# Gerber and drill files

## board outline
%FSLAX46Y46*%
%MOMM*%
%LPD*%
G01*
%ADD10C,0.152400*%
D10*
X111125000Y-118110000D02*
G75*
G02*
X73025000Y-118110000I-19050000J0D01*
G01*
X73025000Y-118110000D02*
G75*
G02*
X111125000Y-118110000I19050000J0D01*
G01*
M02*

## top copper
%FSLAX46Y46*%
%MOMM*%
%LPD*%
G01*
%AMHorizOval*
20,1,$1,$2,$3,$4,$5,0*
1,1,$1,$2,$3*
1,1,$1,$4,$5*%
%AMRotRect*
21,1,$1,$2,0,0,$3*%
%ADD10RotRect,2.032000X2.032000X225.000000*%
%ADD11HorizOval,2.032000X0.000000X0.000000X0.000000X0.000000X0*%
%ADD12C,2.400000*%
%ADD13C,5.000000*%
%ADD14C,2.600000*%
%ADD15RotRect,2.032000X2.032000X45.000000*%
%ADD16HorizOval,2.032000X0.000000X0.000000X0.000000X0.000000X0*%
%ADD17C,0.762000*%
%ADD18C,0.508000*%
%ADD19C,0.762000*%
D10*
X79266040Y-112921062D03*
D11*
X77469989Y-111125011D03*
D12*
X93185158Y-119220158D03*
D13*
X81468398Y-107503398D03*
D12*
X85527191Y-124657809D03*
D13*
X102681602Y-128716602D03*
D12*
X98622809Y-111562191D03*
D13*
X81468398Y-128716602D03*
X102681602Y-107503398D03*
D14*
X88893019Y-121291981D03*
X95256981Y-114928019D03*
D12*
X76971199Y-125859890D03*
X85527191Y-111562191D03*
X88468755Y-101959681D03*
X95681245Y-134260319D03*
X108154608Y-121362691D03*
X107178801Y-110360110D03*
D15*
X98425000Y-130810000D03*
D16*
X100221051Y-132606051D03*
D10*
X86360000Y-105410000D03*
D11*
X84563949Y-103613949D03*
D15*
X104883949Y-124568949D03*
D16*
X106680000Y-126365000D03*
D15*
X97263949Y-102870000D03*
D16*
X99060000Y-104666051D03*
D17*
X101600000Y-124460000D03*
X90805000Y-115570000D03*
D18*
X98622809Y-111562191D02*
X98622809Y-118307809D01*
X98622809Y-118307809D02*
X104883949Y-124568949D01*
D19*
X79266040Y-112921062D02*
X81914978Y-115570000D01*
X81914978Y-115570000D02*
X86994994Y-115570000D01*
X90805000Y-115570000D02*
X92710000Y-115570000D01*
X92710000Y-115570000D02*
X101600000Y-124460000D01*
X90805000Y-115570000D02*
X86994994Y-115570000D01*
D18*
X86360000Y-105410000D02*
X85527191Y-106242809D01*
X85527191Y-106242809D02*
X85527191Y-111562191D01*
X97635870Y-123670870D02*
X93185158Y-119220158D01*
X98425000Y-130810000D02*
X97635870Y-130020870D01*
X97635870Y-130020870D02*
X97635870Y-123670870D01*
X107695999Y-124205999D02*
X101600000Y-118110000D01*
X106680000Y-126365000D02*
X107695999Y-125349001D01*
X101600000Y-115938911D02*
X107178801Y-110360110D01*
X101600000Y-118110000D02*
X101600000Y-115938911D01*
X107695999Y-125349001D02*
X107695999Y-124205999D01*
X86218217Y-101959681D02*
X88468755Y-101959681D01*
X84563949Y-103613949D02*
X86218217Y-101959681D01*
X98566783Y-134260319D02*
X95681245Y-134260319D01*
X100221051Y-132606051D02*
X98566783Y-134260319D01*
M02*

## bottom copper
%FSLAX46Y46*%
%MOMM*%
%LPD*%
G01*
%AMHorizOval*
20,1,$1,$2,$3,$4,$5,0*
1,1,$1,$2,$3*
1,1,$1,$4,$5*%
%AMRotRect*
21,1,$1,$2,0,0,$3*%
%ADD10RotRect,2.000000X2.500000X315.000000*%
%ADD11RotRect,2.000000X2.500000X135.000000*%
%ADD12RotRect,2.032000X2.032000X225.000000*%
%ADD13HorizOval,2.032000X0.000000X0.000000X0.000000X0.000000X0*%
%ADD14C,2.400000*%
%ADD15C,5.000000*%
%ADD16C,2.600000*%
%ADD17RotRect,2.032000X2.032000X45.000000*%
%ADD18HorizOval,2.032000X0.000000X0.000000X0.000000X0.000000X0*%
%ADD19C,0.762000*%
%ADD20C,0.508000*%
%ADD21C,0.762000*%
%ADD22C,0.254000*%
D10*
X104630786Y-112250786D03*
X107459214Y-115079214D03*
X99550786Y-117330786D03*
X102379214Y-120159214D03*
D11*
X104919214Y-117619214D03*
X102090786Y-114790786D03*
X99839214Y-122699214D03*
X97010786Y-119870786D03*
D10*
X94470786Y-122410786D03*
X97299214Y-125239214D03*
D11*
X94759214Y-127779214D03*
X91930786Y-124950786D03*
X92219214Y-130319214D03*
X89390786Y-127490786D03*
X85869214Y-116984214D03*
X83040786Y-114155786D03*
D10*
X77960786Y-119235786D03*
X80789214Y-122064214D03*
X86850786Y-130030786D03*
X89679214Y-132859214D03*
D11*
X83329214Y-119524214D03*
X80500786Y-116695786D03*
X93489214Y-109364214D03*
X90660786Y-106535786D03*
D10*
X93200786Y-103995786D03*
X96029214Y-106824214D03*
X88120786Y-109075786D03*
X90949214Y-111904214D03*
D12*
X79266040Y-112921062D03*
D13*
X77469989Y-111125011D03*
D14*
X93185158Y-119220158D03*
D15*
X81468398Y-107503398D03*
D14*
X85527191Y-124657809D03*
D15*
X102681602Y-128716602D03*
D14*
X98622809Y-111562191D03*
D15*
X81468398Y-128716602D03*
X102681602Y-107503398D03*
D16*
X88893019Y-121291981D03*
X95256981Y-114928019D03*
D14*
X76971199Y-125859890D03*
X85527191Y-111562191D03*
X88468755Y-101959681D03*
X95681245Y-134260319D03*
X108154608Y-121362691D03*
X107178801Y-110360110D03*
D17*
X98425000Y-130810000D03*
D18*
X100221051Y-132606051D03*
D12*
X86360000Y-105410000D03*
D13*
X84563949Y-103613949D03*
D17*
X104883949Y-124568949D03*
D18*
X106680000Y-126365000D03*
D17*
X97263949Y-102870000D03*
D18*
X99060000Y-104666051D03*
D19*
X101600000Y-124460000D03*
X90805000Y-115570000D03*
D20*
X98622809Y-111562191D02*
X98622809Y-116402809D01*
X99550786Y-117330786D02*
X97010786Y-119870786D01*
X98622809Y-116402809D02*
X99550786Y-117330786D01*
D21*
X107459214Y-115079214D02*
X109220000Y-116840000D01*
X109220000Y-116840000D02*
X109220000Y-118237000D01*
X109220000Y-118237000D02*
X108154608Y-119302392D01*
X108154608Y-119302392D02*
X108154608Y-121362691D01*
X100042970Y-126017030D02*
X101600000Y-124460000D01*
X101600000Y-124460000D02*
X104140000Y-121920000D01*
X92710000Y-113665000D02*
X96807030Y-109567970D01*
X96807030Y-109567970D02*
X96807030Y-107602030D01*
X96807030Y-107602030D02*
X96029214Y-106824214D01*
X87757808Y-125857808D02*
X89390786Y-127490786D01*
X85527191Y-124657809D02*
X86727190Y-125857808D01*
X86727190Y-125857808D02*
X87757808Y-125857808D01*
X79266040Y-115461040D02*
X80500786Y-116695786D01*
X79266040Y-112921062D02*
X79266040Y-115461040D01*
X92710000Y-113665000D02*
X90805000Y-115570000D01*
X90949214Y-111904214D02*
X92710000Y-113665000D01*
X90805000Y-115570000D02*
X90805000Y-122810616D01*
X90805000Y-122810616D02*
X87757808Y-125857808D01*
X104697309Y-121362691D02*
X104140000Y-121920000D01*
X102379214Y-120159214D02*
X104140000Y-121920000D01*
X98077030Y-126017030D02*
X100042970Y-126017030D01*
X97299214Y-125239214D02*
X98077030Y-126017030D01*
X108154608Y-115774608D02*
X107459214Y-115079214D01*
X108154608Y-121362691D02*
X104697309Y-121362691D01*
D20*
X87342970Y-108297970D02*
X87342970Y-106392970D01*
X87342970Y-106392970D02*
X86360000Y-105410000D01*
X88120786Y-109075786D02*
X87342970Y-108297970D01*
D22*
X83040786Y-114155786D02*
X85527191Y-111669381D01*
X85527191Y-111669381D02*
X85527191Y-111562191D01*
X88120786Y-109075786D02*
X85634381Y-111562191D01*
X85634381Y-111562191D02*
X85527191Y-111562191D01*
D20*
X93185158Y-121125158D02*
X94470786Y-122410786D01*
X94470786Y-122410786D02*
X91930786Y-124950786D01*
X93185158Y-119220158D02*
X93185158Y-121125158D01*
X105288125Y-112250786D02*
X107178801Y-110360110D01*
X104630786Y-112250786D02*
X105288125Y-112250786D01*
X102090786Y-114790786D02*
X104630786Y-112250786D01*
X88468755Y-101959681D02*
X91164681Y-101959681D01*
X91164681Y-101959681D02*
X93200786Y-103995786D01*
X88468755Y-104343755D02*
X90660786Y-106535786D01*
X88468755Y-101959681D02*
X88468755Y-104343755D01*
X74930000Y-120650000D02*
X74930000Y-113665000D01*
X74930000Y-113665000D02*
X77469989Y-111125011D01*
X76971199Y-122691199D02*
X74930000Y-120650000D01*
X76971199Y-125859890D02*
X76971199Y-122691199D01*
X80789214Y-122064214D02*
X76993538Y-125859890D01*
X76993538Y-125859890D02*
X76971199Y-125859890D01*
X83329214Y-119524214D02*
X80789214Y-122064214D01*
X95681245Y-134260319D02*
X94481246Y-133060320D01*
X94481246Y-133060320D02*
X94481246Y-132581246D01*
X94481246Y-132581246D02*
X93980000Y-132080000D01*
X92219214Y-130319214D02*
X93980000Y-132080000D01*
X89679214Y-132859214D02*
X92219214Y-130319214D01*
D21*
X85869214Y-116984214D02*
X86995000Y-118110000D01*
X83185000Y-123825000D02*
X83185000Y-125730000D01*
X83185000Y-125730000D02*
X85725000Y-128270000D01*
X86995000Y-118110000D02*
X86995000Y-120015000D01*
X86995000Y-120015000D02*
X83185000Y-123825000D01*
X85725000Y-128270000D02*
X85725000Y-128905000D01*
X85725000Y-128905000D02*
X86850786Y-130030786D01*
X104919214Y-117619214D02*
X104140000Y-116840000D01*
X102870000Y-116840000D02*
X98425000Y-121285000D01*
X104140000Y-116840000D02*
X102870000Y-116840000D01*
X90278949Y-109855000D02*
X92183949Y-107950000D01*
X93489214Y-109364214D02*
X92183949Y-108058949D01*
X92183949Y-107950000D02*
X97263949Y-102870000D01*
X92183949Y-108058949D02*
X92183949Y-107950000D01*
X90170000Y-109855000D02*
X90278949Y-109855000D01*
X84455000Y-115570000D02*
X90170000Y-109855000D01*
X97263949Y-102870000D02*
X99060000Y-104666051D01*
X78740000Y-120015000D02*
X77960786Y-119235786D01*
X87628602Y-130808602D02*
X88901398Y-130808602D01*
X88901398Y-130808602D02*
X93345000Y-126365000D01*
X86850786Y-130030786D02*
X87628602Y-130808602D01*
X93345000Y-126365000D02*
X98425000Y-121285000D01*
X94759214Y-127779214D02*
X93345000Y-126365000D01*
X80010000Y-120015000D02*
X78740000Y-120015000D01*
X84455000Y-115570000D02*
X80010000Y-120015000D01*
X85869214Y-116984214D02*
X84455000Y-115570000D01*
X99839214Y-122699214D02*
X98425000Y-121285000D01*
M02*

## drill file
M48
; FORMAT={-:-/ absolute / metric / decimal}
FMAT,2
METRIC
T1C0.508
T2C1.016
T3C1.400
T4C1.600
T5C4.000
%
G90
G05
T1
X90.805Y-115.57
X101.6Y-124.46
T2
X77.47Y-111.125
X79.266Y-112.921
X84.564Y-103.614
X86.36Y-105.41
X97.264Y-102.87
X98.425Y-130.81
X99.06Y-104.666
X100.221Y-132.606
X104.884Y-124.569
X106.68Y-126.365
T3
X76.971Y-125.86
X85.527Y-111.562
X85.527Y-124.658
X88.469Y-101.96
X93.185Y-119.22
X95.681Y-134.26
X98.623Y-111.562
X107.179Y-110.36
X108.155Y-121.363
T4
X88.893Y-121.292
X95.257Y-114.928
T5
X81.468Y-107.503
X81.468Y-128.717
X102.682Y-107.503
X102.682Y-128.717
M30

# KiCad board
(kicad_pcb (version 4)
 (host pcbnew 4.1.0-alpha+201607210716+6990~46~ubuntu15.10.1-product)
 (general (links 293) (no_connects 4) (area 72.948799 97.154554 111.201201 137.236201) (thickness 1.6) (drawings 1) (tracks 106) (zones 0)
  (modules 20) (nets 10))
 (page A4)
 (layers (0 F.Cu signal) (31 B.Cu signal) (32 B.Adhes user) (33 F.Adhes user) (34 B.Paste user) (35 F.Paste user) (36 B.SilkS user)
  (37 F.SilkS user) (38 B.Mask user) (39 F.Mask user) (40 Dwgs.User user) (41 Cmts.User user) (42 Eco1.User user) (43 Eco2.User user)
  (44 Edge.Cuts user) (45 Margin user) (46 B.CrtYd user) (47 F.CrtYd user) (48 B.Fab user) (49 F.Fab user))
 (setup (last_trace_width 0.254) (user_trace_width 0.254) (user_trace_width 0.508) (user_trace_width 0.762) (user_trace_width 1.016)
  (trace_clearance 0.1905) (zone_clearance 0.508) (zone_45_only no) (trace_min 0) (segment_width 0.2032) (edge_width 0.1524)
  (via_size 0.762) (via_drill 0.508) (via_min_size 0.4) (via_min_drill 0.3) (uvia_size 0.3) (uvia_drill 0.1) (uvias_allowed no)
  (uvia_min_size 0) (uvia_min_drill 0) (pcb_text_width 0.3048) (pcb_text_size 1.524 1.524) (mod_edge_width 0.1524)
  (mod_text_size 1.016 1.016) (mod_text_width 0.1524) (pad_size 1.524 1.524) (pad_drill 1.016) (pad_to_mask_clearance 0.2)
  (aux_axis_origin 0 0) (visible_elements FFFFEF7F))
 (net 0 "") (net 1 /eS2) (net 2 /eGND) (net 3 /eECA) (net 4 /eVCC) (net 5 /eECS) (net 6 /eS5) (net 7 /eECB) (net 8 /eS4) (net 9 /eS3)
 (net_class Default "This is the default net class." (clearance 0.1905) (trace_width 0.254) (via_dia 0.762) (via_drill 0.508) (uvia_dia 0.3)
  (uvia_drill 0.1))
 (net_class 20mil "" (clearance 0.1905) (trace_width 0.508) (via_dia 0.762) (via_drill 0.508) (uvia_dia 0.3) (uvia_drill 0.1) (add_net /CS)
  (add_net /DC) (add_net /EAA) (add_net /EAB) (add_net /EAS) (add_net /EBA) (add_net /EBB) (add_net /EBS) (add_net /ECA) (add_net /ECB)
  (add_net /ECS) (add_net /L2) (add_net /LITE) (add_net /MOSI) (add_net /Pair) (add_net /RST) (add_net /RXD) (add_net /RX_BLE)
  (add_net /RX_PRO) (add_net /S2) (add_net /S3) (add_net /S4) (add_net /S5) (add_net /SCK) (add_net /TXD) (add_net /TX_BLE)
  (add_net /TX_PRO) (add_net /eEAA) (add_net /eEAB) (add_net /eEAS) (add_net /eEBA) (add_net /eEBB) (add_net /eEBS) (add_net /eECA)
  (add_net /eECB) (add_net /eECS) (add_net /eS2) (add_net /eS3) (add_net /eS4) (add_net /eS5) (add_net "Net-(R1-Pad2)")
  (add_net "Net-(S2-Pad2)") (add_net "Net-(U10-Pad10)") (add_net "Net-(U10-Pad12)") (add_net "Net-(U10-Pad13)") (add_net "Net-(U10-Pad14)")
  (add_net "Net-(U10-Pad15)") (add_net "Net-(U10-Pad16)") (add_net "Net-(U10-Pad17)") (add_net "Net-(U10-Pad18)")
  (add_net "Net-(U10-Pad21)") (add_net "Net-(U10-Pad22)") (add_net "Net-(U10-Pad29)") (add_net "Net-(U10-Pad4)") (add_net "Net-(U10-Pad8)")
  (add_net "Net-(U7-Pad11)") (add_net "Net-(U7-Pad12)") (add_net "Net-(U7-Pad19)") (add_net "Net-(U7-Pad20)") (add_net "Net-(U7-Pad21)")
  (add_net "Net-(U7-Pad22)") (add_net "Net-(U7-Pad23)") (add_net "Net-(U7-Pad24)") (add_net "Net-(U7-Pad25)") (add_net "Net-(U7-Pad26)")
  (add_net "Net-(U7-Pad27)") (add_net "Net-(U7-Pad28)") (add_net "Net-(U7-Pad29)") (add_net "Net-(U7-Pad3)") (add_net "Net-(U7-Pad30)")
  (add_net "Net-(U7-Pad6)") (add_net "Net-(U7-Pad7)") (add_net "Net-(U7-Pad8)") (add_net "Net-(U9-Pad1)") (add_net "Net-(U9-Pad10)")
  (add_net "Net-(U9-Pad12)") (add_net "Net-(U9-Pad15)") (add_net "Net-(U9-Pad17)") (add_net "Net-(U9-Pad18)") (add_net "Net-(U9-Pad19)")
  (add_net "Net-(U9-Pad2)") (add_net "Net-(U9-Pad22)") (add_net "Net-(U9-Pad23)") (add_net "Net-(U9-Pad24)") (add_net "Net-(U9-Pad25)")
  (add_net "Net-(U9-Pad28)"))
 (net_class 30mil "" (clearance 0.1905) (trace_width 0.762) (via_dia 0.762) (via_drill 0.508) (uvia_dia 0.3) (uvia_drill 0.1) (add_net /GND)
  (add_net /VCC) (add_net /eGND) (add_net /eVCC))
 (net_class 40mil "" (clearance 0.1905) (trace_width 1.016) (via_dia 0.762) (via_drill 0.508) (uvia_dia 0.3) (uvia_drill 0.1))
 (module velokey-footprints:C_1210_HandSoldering (layer B.Cu) (at 106.045 113.665 315)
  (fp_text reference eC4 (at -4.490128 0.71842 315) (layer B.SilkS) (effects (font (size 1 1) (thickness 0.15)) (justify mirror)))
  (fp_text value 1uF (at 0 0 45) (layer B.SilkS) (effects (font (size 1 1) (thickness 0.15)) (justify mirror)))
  (pad 1 smd rect (at -2 0 315) (size 2 2.5) (layers B.Cu B.Paste B.Mask) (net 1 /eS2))
  (pad 2 smd rect (at 2 0 315) (size 2 2.5) (layers B.Cu B.Paste B.Mask) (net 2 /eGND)))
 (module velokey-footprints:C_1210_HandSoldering (layer B.Cu) (at 100.965 118.745 315)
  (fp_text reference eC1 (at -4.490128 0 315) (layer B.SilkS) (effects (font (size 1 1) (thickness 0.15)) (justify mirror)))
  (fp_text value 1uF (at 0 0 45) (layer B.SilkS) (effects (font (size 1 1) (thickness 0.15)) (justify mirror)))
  (pad 1 smd rect (at -2 0 315) (size 2 2.5) (layers B.Cu B.Paste B.Mask) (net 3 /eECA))
  (pad 2 smd rect (at 2 0 315) (size 2 2.5) (layers B.Cu B.Paste B.Mask) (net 2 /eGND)))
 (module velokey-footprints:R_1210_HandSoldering (layer B.Cu) (at 103.505 116.205 135)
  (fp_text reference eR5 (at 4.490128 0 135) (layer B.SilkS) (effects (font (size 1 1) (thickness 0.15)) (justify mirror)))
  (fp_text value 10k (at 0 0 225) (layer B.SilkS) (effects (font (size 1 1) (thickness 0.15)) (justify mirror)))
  (pad 1 smd rect (at -2 0 135) (size 2 2.5) (layers B.Cu B.Paste B.Mask) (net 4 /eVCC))
  (pad 2 smd rect (at 2 0 135) (size 2 2.5) (layers B.Cu B.Paste B.Mask) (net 1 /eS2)))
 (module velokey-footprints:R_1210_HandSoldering (layer B.Cu) (at 98.425 121.285 135)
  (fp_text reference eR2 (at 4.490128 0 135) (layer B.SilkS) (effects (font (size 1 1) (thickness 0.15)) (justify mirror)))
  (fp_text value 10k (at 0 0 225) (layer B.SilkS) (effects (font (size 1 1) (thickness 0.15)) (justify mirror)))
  (pad 1 smd rect (at -2 0 135) (size 2 2.5) (layers B.Cu B.Paste B.Mask) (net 4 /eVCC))
  (pad 2 smd rect (at 2 0 135) (size 2 2.5) (layers B.Cu B.Paste B.Mask) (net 3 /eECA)))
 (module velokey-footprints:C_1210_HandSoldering (layer B.Cu) (at 95.885 123.825 315)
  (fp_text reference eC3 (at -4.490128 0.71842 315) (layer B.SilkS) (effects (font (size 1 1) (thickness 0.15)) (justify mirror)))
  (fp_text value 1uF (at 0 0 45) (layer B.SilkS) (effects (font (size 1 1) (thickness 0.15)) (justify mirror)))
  (pad 1 smd rect (at -2 0 315) (size 2 2.5) (layers B.Cu B.Paste B.Mask) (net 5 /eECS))
  (pad 2 smd rect (at 2 0 315) (size 2 2.5) (layers B.Cu B.Paste B.Mask) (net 2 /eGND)))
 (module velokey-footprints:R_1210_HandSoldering (layer B.Cu) (at 93.345 126.365 135)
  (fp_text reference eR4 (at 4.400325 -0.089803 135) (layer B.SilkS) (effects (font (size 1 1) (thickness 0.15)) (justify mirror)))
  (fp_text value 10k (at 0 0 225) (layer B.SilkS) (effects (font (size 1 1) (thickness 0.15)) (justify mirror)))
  (pad 1 smd rect (at -2 0 135) (size 2 2.5) (layers B.Cu B.Paste B.Mask) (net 4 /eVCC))
  (pad 2 smd rect (at 2 0 135) (size 2 2.5) (layers B.Cu B.Paste B.Mask) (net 5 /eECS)))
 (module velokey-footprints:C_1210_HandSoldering (layer B.Cu) (at 90.805 128.905 135)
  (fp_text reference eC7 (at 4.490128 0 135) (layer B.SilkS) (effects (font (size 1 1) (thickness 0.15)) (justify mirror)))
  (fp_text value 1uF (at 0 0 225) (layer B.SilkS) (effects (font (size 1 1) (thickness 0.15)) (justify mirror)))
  (pad 1 smd rect (at -2 0 135) (size 2 2.5) (layers B.Cu B.Paste B.Mask) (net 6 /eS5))
  (pad 2 smd rect (at 2 0 135) (size 2 2.5) (layers B.Cu B.Paste B.Mask) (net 2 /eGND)))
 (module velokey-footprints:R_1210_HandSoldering (layer B.Cu) (at 84.455 115.57 135)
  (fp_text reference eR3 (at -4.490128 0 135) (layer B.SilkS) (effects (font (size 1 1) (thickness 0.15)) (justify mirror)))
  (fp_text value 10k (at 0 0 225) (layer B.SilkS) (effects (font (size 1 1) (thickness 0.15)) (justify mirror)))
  (pad 1 smd rect (at -2 0 135) (size 2 2.5) (layers B.Cu B.Paste B.Mask) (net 4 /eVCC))
  (pad 2 smd rect (at 2 0 135) (size 2 2.5) (layers B.Cu B.Paste B.Mask) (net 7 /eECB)))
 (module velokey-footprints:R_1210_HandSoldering (layer B.Cu) (at 79.375 120.65 315)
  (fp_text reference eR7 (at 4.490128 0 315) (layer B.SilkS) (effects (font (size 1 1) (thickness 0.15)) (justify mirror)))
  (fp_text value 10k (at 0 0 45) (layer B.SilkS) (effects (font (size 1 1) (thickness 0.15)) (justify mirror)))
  (pad 1 smd rect (at -2 0 315) (size 2 2.5) (layers B.Cu B.Paste B.Mask) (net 4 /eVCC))
  (pad 2 smd rect (at 2 0 315) (size 2 2.5) (layers B.Cu B.Paste B.Mask) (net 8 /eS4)))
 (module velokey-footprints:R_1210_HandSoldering (layer B.Cu) (at 88.265 131.445 315)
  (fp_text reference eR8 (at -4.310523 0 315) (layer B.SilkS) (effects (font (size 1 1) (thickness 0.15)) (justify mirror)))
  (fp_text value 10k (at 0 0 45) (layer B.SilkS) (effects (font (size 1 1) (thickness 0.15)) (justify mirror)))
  (pad 1 smd rect (at -2 0 315) (size 2 2.5) (layers B.Cu B.Paste B.Mask) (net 4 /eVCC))
  (pad 2 smd rect (at 2 0 315) (size 2 2.5) (layers B.Cu B.Paste B.Mask) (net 6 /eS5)))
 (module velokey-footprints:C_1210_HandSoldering (layer B.Cu) (at 81.915 118.11 135)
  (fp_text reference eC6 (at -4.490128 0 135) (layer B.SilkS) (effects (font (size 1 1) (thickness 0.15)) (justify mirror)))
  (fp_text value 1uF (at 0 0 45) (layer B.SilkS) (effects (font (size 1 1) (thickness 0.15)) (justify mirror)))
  (pad 1 smd rect (at -2 0 135) (size 2 2.5) (layers B.Cu B.Paste B.Mask) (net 8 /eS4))
  (pad 2 smd rect (at 2 0 135) (size 2 2.5) (layers B.Cu B.Paste B.Mask) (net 2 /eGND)))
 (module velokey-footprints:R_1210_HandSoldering (layer B.Cu) (at 92.075 107.95 135)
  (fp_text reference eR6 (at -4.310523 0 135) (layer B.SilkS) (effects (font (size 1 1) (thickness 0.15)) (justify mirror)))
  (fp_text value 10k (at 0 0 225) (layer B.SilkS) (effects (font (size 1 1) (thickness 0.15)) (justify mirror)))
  (pad 1 smd rect (at -2 0 135) (size 2 2.5) (layers B.Cu B.Paste B.Mask) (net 4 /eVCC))
  (pad 2 smd rect (at 2 0 135) (size 2 2.5) (layers B.Cu B.Paste B.Mask) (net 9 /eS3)))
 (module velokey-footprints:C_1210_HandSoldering (layer B.Cu) (at 94.615 105.41 315)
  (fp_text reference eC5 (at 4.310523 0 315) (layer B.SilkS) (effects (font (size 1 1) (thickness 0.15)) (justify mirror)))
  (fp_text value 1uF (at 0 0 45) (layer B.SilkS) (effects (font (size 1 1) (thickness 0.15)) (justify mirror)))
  (pad 1 smd rect (at -2 0 315) (size 2 2.5) (layers B.Cu B.Paste B.Mask) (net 9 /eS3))
  (pad 2 smd rect (at 2 0 315) (size 2 2.5) (layers B.Cu B.Paste B.Mask) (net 2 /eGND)))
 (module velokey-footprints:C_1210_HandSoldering (layer B.Cu) (at 89.535 110.49 315)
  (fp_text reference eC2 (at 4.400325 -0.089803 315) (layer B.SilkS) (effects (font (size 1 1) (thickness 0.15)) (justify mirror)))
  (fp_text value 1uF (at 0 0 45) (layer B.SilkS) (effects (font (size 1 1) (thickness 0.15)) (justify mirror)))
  (pad 1 smd rect (at -2 0 315) (size 2 2.5) (layers B.Cu B.Paste B.Mask) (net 7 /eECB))
  (pad 2 smd rect (at 2 0 315) (size 2 2.5) (layers B.Cu B.Paste B.Mask) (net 2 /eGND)))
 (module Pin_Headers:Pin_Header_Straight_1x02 (layer F.Cu) (at 79.26604 112.921062 225)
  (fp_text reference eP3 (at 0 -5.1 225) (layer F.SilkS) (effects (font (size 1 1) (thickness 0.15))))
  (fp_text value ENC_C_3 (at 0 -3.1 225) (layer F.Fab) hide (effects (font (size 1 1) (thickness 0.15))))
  (pad 1 thru_hole rect (at 0 0 225) (size 2.032 2.032) (drill 1.016) (layers *.Cu *.Mask F.SilkS) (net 2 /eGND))
  (pad 2 thru_hole oval (at 0 2.54 225) (size 2.032 2.032) (drill 1.016) (layers *.Cu *.Mask F.SilkS) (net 8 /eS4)))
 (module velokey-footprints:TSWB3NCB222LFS (layer F.Cu) (at 92.075 118.11 45)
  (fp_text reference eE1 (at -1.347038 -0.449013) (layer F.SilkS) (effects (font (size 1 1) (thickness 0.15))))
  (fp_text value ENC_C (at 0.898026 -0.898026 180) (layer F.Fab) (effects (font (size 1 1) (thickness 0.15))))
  (pad 4 thru_hole circle (at 0 1.57 45) (size 2.4 2.4) (drill 1.4) (layers *.Cu *.Mask F.SilkS) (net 5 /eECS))
  (pad 12 thru_hole circle (at 0 -15 45) (size 5 5) (drill 4) (layers *.Cu *.Mask F.SilkS))
  (pad 2 thru_hole circle (at -9.26 0 45) (size 2.4 2.4) (drill 1.4) (layers *.Cu *.Mask F.SilkS) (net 2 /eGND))
  (pad 14 thru_hole circle (at 0 15 45) (size 5 5) (drill 4) (layers *.Cu *.Mask F.SilkS))
  (pad 1 thru_hole circle (at 9.26 0 45) (size 2.4 2.4) (drill 1.4) (layers *.Cu *.Mask F.SilkS) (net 3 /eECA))
  (pad 13 thru_hole circle (at -15 0 45) (size 5 5) (drill 4) (layers *.Cu *.Mask F.SilkS))
  (pad 15 thru_hole circle (at 15 0 45) (size 5 5) (drill 4) (layers *.Cu *.Mask F.SilkS))
  (pad 5 thru_hole circle (at -4.5 0 45) (size 2.6 2.6) (drill 1.6) (layers *.Cu *.Mask F.SilkS))
  (pad 6 thru_hole circle (at 4.5 0 45) (size 2.6 2.6) (drill 1.6) (layers *.Cu *.Mask F.SilkS))
  (pad 9 thru_hole circle (at -16.16 -5.2 45) (size 2.4 2.4) (drill 1.4) (layers *.Cu *.Mask F.SilkS) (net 8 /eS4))
  (pad 3 thru_hole circle (at 0 -9.26 45) (size 2.4 2.4) (drill 1.4) (layers *.Cu *.Mask F.SilkS) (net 7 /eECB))
  (pad 8 thru_hole circle (at 8.87 -13.97 45) (size 2.4 2.4) (drill 1.4) (layers *.Cu *.Mask F.SilkS) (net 9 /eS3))
  (pad 10 thru_hole circle (at -8.87 13.97 45) (size 2.4 2.4) (drill 1.4) (layers *.Cu *.Mask F.SilkS) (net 6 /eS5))
  (pad 11 thru_hole circle (at 9.07 13.67 45) (size 2.4 2.4) (drill 1.4) (layers *.Cu *.Mask F.SilkS) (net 2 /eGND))
  (pad 7 thru_hole circle (at 16.16 5.2 45) (size 2.4 2.4) (drill 1.4) (layers *.Cu *.Mask F.SilkS) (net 1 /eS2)))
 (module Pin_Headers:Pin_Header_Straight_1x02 (layer F.Cu) (at 98.425 130.81 45)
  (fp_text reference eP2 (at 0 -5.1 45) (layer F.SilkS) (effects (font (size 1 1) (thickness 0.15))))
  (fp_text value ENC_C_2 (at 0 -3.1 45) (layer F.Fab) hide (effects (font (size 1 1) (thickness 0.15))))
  (pad 1 thru_hole rect (at 0 0 45) (size 2.032 2.032) (drill 1.016) (layers *.Cu *.Mask F.SilkS) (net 5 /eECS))
  (pad 2 thru_hole oval (at 0 2.54 45) (size 2.032 2.032) (drill 1.016) (layers *.Cu *.Mask F.SilkS) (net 6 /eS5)))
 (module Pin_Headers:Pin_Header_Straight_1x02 (layer F.Cu) (at 86.36 105.41 225)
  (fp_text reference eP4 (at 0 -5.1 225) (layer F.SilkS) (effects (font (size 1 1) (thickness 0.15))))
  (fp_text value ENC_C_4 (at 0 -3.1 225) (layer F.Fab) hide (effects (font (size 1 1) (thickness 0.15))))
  (pad 1 thru_hole rect (at 0 0 225) (size 2.032 2.032) (drill 1.016) (layers *.Cu *.Mask F.SilkS) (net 7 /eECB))
  (pad 2 thru_hole oval (at 0 2.54 225) (size 2.032 2.032) (drill 1.016) (layers *.Cu *.Mask F.SilkS) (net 9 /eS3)))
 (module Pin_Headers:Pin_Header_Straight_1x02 (layer F.Cu) (at 104.883949 124.568949 45)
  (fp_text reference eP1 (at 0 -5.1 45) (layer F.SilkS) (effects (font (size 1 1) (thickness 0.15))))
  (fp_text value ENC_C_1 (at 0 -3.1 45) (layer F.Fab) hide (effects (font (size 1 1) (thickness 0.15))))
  (pad 1 thru_hole rect (at 0 0 45) (size 2.032 2.032) (drill 1.016) (layers *.Cu *.Mask F.SilkS) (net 3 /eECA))
  (pad 2 thru_hole oval (at 0 2.54 45) (size 2.032 2.032) (drill 1.016) (layers *.Cu *.Mask F.SilkS) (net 1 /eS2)))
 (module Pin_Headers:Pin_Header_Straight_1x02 (layer F.Cu) (at 97.263949 102.87 45)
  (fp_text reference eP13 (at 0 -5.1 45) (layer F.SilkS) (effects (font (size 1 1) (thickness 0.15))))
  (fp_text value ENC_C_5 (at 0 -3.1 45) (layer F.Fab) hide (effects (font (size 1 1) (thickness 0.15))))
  (pad 1 thru_hole rect (at 0 0 45) (size 2.032 2.032) (drill 1.016) (layers *.Cu *.Mask F.SilkS) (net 4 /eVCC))
  (pad 2 thru_hole oval (at 0 2.54 45) (size 2.032 2.032) (drill 1.016) (layers *.Cu *.Mask F.SilkS) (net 4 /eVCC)))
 (gr_circle (center 92.075 118.11) (end 111.125 118.11) (layer Edge.Cuts) (width 0.1524))
 (segment (start 98.622809 111.562191) (end 98.622809 116.402809) (width 0.508) (layer B.Cu) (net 3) (status 10))
 (segment (start 99.550786 117.330786) (end 97.010786 119.870786) (width 0.508) (layer B.Cu) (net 3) (status 30))
 (segment (start 98.622809 116.402809) (end 99.550786 117.330786) (width 0.508) (layer B.Cu) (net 3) (status 20))
 (segment (start 98.622809 111.562191) (end 98.622809 118.307809) (width 0.508) (layer F.Cu) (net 3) (status 10))
 (segment (start 98.622809 118.307809) (end 104.883949 124.568949) (width 0.508) (layer F.Cu) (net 3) (status 20))
 (segment (start 107.459214 115.079214) (end 109.22 116.84) (width 0.762) (layer B.Cu) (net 2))
 (segment (start 109.22 116.84) (end 109.22 118.237) (width 0.762) (layer B.Cu) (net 2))
 (segment (start 109.22 118.237) (end 108.154608 119.302392) (width 0.762) (layer B.Cu) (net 2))
 (segment (start 108.154608 119.302392) (end 108.154608 121.362691) (width 0.762) (layer B.Cu) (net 2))
 (segment (start 79.26604 112.921062) (end 81.914978 115.57) (width 0.762) (layer F.Cu) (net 2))
 (segment (start 81.914978 115.57) (end 86.994994 115.57) (width 0.762) (layer F.Cu) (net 2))
 (segment (start 100.04297 126.01703) (end 101.6 124.46) (width 0.762) (layer B.Cu) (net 2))
 (segment (start 101.6 124.46) (end 104.14 121.92) (width 0.762) (layer B.Cu) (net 2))
 (segment (start 90.805 115.57) (end 92.71 115.57) (width 0.762) (layer F.Cu) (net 2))
 (segment (start 92.71 115.57) (end 101.6 124.46) (width 0.762) (layer F.Cu) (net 2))
 (via (at 101.6 124.46) (size 0.762) (drill 0.508) (layers F.Cu B.Cu) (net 2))
 (segment (start 92.71 113.665) (end 96.80703 109.56797) (width 0.762) (layer B.Cu) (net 2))
 (segment (start 96.80703 109.56797) (end 96.80703 107.60203) (width 0.762) (layer B.Cu) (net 2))
 (segment (start 96.80703 107.60203) (end 96.029214 106.824214) (width 0.762) (layer B.Cu) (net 2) (status 20))
 (segment (start 87.757808 125.857808) (end 89.390786 127.490786) (width 0.762) (layer B.Cu) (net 2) (status 20))
 (segment (start 85.527191 124.657809) (end 86.72719 125.857808) (width 0.762) (layer B.Cu) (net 2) (status 10))
 (segment (start 86.72719 125.857808) (end 87.757808 125.857808) (width 0.762) (layer B.Cu) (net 2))
 (segment (start 79.26604 115.46104) (end 80.500786 116.695786) (width 0.762) (layer B.Cu) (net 2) (status 20))
 (segment (start 79.26604 112.921062) (end 79.26604 115.46104) (width 0.762) (layer B.Cu) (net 2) (status 10))
 (segment (start 92.71 113.665) (end 90.805 115.57) (width 0.762) (layer B.Cu) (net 2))
 (segment (start 90.949214 111.904214) (end 92.71 113.665) (width 0.762) (layer B.Cu) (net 2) (status 10))
 (segment (start 90.805 115.57) (end 90.805 122.810616) (width 0.762) (layer B.Cu) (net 2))
 (segment (start 90.805 122.810616) (end 87.757808 125.857808) (width 0.762) (layer B.Cu) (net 2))
 (segment (start 104.697309 121.362691) (end 104.14 121.92) (width 0.762) (layer B.Cu) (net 2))
 (segment (start 102.379214 120.159214) (end 104.14 121.92) (width 0.762) (layer B.Cu) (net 2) (status 10))
 (segment (start 98.07703 126.01703) (end 100.04297 126.01703) (width 0.762) (layer B.Cu) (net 2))
 (segment (start 97.299214 125.239214) (end 98.07703 126.01703) (width 0.762) (layer B.Cu) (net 2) (status 10))
 (segment (start 108.154608 115.774608) (end 107.459214 115.079214) (width 0.762) (layer B.Cu) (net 2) (status 30))
 (segment (start 108.154608 121.362691) (end 104.697309 121.362691) (width 0.762) (layer B.Cu) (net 2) (status 10))
 (segment (start 90.805 115.57) (end 86.994994 115.57) (width 0.762) (layer F.Cu) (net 2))
 (via (at 90.805 115.57) (size 0.762) (drill 0.508) (layers F.Cu B.Cu) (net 2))
 (segment (start 87.34297 108.29797) (end 87.34297 106.39297) (width 0.508) (layer B.Cu) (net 7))
 (segment (start 87.34297 106.39297) (end 86.36 105.41) (width 0.508) (layer B.Cu) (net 7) (status 20))
 (segment (start 88.120786 109.075786) (end 87.34297 108.29797) (width 0.508) (layer B.Cu) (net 7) (status 10))
 (segment (start 83.040786 114.155786) (end 85.527191 111.669381) (width 0.254) (layer B.Cu) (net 7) (status 30))
 (segment (start 85.527191 111.669381) (end 85.527191 111.562191) (width 0.254) (layer B.Cu) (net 7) (status 30))
 (segment (start 88.120786 109.075786) (end 85.634381 111.562191) (width 0.254) (layer B.Cu) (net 7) (status 30))
 (segment (start 85.634381 111.562191) (end 85.527191 111.562191) (width 0.254) (layer B.Cu) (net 7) (status 30))
 (segment (start 86.36 105.41) (end 85.527191 106.242809) (width 0.508) (layer F.Cu) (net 7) (status 10))
 (segment (start 85.527191 106.242809) (end 85.527191 111.562191) (width 0.508) (layer F.Cu) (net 7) (status 20))
 (segment (start 93.185158 121.125158) (end 94.470786 122.410786) (width 0.508) (layer B.Cu) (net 5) (status 20))
 (segment (start 94.470786 122.410786) (end 91.930786 124.950786) (width 0.508) (layer B.Cu) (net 5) (status 30))
 (segment (start 93.185158 119.220158) (end 93.185158 121.125158) (width 0.508) (layer B.Cu) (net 5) (status 10))
 (segment (start 97.63587 123.67087) (end 93.185158 119.220158) (width 0.508) (layer F.Cu) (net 5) (status 20))
 (segment (start 98.425 130.81) (end 97.63587 130.02087) (width 0.508) (layer F.Cu) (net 5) (status 10))
 (segment (start 97.63587 130.02087) (end 97.63587 123.67087) (width 0.508) (layer F.Cu) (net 5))
 (segment (start 105.288125 112.250786) (end 107.178801 110.36011) (width 0.508) (layer B.Cu) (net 1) (status 30))
 (segment (start 104.630786 112.250786) (end 105.288125 112.250786) (width 0.508) (layer B.Cu) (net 1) (status 30))
 (segment (start 102.090786 114.790786) (end 104.630786 112.250786) (width 0.508) (layer B.Cu) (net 1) (status 30))
 (segment (start 107.695999 124.205999) (end 101.6 118.11) (width 0.508) (layer F.Cu) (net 1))
 (segment (start 106.68 126.365) (end 107.695999 125.349001) (width 0.508) (layer F.Cu) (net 1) (status 10))
 (segment (start 101.6 115.938911) (end 107.178801 110.36011) (width 0.508) (layer F.Cu) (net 1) (status 20))
 (segment (start 101.6 118.11) (end 101.6 115.938911) (width 0.508) (layer F.Cu) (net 1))
 (segment (start 107.695999 125.349001) (end 107.695999 124.205999) (width 0.508) (layer F.Cu) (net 1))
 (segment (start 88.468755 101.959681) (end 91.164681 101.959681) (width 0.508) (layer B.Cu) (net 9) (status 10))
 (segment (start 91.164681 101.959681) (end 93.200786 103.995786) (width 0.508) (layer B.Cu) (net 9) (status 20))
 (segment (start 88.468755 104.343755) (end 90.660786 106.535786) (width 0.508) (layer B.Cu) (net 9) (status 20))
 (segment (start 88.468755 101.959681) (end 88.468755 104.343755) (width 0.508) (layer B.Cu) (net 9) (status 10))
 (segment (start 86.218217 101.959681) (end 88.468755 101.959681) (width 0.508) (layer F.Cu) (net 9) (status 20))
 (segment (start 84.563949 103.613949) (end 86.218217 101.959681) (width 0.508) (layer F.Cu) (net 9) (status 10))
 (segment (start 74.93 120.65) (end 74.93 113.665) (width 0.508) (layer B.Cu) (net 8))
 (segment (start 74.93 113.665) (end 77.469989 111.125011) (width 0.508) (layer B.Cu) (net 8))
 (segment (start 76.971199 122.691199) (end 74.93 120.65) (width 0.508) (layer B.Cu) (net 8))
 (segment (start 76.971199 125.85989) (end 76.971199 122.691199) (width 0.508) (layer B.Cu) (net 8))
 (segment (start 80.789214 122.064214) (end 76.993538 125.85989) (width 0.508) (layer B.Cu) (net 8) (status 30))
 (segment (start 76.993538 125.85989) (end 76.971199 125.85989) (width 0.508) (layer B.Cu) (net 8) (status 30))
 (segment (start 83.329214 119.524214) (end 80.789214 122.064214) (width 0.508) (layer B.Cu) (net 8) (status 30))
 (segment (start 95.681245 134.260319) (end 94.481246 133.06032) (width 0.508) (layer B.Cu) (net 6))
 (segment (start 94.481246 133.06032) (end 94.481246 132.581246) (width 0.508) (layer B.Cu) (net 6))
 (segment (start 94.481246 132.581246) (end 93.98 132.08) (width 0.508) (layer B.Cu) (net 6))
 (segment (start 92.219214 130.319214) (end 93.98 132.08) (width 0.508) (layer B.Cu) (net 6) (status 10))
 (segment (start 89.679214 132.859214) (end 92.219214 130.319214) (width 0.508) (layer B.Cu) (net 6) (status 30))
 (segment (start 98.566783 134.260319) (end 95.681245 134.260319) (width 0.508) (layer F.Cu) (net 6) (status 20))
 (segment (start 100.221051 132.606051) (end 98.566783 134.260319) (width 0.508) (layer F.Cu) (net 6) (status 10))
 (segment (start 85.869214 116.984214) (end 86.995 118.11) (width 0.762) (layer B.Cu) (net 4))
 (segment (start 83.185 123.825) (end 83.185 125.73) (width 0.762) (layer B.Cu) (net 4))
 (segment (start 83.185 125.73) (end 85.725 128.27) (width 0.762) (layer B.Cu) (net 4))
 (segment (start 86.995 118.11) (end 86.995 120.015) (width 0.762) (layer B.Cu) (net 4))
 (segment (start 86.995 120.015) (end 83.185 123.825) (width 0.762) (layer B.Cu) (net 4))
 (segment (start 85.725 128.27) (end 85.725 128.905) (width 0.762) (layer B.Cu) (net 4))
 (segment (start 85.725 128.905) (end 86.850786 130.030786) (width 0.762) (layer B.Cu) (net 4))
 (segment (start 104.919214 117.619214) (end 104.14 116.84) (width 0.762) (layer B.Cu) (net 4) (status 10))
 (segment (start 102.87 116.84) (end 98.425 121.285) (width 0.762) (layer B.Cu) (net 4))
 (segment (start 104.14 116.84) (end 102.87 116.84) (width 0.762) (layer B.Cu) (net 4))
 (segment (start 90.278949 109.855) (end 92.183949 107.95) (width 0.762) (layer B.Cu) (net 4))
 (segment (start 93.489214 109.364214) (end 92.183949 108.058949) (width 0.762) (layer B.Cu) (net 4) (status 10))
 (segment (start 92.183949 107.95) (end 97.263949 102.87) (width 0.762) (layer B.Cu) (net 4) (status 20))
 (segment (start 92.183949 108.058949) (end 92.183949 107.95) (width 0.762) (layer B.Cu) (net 4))
 (segment (start 90.17 109.855) (end 90.278949 109.855) (width 0.762) (layer B.Cu) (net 4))
 (segment (start 84.455 115.57) (end 90.17 109.855) (width 0.762) (layer B.Cu) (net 4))
 (segment (start 97.263949 102.87) (end 99.06 104.666051) (width 0.762) (layer B.Cu) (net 4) (status 30))
 (segment (start 78.74 120.015) (end 77.960786 119.235786) (width 0.762) (layer B.Cu) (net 4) (status 20))
 (segment (start 87.628602 130.808602) (end 88.901398 130.808602) (width 0.762) (layer B.Cu) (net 4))
 (segment (start 88.901398 130.808602) (end 93.345 126.365) (width 0.762) (layer B.Cu) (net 4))
 (segment (start 86.850786 130.030786) (end 87.628602 130.808602) (width 0.762) (layer B.Cu) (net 4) (status 10))
 (segment (start 93.345 126.365) (end 98.425 121.285) (width 0.762) (layer B.Cu) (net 4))
 (segment (start 94.759214 127.779214) (end 93.345 126.365) (width 0.762) (layer B.Cu) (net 4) (status 10))
 (segment (start 80.01 120.015) (end 78.74 120.015) (width 0.762) (layer B.Cu) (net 4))
 (segment (start 84.455 115.57) (end 80.01 120.015) (width 0.762) (layer B.Cu) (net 4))
 (segment (start 85.869214 116.984214) (end 84.455 115.57) (width 0.762) (layer B.Cu) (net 4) (status 10))
 (segment (start 99.839214 122.699214) (end 98.425 121.285) (width 0.762) (layer B.Cu) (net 4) (status 10)))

